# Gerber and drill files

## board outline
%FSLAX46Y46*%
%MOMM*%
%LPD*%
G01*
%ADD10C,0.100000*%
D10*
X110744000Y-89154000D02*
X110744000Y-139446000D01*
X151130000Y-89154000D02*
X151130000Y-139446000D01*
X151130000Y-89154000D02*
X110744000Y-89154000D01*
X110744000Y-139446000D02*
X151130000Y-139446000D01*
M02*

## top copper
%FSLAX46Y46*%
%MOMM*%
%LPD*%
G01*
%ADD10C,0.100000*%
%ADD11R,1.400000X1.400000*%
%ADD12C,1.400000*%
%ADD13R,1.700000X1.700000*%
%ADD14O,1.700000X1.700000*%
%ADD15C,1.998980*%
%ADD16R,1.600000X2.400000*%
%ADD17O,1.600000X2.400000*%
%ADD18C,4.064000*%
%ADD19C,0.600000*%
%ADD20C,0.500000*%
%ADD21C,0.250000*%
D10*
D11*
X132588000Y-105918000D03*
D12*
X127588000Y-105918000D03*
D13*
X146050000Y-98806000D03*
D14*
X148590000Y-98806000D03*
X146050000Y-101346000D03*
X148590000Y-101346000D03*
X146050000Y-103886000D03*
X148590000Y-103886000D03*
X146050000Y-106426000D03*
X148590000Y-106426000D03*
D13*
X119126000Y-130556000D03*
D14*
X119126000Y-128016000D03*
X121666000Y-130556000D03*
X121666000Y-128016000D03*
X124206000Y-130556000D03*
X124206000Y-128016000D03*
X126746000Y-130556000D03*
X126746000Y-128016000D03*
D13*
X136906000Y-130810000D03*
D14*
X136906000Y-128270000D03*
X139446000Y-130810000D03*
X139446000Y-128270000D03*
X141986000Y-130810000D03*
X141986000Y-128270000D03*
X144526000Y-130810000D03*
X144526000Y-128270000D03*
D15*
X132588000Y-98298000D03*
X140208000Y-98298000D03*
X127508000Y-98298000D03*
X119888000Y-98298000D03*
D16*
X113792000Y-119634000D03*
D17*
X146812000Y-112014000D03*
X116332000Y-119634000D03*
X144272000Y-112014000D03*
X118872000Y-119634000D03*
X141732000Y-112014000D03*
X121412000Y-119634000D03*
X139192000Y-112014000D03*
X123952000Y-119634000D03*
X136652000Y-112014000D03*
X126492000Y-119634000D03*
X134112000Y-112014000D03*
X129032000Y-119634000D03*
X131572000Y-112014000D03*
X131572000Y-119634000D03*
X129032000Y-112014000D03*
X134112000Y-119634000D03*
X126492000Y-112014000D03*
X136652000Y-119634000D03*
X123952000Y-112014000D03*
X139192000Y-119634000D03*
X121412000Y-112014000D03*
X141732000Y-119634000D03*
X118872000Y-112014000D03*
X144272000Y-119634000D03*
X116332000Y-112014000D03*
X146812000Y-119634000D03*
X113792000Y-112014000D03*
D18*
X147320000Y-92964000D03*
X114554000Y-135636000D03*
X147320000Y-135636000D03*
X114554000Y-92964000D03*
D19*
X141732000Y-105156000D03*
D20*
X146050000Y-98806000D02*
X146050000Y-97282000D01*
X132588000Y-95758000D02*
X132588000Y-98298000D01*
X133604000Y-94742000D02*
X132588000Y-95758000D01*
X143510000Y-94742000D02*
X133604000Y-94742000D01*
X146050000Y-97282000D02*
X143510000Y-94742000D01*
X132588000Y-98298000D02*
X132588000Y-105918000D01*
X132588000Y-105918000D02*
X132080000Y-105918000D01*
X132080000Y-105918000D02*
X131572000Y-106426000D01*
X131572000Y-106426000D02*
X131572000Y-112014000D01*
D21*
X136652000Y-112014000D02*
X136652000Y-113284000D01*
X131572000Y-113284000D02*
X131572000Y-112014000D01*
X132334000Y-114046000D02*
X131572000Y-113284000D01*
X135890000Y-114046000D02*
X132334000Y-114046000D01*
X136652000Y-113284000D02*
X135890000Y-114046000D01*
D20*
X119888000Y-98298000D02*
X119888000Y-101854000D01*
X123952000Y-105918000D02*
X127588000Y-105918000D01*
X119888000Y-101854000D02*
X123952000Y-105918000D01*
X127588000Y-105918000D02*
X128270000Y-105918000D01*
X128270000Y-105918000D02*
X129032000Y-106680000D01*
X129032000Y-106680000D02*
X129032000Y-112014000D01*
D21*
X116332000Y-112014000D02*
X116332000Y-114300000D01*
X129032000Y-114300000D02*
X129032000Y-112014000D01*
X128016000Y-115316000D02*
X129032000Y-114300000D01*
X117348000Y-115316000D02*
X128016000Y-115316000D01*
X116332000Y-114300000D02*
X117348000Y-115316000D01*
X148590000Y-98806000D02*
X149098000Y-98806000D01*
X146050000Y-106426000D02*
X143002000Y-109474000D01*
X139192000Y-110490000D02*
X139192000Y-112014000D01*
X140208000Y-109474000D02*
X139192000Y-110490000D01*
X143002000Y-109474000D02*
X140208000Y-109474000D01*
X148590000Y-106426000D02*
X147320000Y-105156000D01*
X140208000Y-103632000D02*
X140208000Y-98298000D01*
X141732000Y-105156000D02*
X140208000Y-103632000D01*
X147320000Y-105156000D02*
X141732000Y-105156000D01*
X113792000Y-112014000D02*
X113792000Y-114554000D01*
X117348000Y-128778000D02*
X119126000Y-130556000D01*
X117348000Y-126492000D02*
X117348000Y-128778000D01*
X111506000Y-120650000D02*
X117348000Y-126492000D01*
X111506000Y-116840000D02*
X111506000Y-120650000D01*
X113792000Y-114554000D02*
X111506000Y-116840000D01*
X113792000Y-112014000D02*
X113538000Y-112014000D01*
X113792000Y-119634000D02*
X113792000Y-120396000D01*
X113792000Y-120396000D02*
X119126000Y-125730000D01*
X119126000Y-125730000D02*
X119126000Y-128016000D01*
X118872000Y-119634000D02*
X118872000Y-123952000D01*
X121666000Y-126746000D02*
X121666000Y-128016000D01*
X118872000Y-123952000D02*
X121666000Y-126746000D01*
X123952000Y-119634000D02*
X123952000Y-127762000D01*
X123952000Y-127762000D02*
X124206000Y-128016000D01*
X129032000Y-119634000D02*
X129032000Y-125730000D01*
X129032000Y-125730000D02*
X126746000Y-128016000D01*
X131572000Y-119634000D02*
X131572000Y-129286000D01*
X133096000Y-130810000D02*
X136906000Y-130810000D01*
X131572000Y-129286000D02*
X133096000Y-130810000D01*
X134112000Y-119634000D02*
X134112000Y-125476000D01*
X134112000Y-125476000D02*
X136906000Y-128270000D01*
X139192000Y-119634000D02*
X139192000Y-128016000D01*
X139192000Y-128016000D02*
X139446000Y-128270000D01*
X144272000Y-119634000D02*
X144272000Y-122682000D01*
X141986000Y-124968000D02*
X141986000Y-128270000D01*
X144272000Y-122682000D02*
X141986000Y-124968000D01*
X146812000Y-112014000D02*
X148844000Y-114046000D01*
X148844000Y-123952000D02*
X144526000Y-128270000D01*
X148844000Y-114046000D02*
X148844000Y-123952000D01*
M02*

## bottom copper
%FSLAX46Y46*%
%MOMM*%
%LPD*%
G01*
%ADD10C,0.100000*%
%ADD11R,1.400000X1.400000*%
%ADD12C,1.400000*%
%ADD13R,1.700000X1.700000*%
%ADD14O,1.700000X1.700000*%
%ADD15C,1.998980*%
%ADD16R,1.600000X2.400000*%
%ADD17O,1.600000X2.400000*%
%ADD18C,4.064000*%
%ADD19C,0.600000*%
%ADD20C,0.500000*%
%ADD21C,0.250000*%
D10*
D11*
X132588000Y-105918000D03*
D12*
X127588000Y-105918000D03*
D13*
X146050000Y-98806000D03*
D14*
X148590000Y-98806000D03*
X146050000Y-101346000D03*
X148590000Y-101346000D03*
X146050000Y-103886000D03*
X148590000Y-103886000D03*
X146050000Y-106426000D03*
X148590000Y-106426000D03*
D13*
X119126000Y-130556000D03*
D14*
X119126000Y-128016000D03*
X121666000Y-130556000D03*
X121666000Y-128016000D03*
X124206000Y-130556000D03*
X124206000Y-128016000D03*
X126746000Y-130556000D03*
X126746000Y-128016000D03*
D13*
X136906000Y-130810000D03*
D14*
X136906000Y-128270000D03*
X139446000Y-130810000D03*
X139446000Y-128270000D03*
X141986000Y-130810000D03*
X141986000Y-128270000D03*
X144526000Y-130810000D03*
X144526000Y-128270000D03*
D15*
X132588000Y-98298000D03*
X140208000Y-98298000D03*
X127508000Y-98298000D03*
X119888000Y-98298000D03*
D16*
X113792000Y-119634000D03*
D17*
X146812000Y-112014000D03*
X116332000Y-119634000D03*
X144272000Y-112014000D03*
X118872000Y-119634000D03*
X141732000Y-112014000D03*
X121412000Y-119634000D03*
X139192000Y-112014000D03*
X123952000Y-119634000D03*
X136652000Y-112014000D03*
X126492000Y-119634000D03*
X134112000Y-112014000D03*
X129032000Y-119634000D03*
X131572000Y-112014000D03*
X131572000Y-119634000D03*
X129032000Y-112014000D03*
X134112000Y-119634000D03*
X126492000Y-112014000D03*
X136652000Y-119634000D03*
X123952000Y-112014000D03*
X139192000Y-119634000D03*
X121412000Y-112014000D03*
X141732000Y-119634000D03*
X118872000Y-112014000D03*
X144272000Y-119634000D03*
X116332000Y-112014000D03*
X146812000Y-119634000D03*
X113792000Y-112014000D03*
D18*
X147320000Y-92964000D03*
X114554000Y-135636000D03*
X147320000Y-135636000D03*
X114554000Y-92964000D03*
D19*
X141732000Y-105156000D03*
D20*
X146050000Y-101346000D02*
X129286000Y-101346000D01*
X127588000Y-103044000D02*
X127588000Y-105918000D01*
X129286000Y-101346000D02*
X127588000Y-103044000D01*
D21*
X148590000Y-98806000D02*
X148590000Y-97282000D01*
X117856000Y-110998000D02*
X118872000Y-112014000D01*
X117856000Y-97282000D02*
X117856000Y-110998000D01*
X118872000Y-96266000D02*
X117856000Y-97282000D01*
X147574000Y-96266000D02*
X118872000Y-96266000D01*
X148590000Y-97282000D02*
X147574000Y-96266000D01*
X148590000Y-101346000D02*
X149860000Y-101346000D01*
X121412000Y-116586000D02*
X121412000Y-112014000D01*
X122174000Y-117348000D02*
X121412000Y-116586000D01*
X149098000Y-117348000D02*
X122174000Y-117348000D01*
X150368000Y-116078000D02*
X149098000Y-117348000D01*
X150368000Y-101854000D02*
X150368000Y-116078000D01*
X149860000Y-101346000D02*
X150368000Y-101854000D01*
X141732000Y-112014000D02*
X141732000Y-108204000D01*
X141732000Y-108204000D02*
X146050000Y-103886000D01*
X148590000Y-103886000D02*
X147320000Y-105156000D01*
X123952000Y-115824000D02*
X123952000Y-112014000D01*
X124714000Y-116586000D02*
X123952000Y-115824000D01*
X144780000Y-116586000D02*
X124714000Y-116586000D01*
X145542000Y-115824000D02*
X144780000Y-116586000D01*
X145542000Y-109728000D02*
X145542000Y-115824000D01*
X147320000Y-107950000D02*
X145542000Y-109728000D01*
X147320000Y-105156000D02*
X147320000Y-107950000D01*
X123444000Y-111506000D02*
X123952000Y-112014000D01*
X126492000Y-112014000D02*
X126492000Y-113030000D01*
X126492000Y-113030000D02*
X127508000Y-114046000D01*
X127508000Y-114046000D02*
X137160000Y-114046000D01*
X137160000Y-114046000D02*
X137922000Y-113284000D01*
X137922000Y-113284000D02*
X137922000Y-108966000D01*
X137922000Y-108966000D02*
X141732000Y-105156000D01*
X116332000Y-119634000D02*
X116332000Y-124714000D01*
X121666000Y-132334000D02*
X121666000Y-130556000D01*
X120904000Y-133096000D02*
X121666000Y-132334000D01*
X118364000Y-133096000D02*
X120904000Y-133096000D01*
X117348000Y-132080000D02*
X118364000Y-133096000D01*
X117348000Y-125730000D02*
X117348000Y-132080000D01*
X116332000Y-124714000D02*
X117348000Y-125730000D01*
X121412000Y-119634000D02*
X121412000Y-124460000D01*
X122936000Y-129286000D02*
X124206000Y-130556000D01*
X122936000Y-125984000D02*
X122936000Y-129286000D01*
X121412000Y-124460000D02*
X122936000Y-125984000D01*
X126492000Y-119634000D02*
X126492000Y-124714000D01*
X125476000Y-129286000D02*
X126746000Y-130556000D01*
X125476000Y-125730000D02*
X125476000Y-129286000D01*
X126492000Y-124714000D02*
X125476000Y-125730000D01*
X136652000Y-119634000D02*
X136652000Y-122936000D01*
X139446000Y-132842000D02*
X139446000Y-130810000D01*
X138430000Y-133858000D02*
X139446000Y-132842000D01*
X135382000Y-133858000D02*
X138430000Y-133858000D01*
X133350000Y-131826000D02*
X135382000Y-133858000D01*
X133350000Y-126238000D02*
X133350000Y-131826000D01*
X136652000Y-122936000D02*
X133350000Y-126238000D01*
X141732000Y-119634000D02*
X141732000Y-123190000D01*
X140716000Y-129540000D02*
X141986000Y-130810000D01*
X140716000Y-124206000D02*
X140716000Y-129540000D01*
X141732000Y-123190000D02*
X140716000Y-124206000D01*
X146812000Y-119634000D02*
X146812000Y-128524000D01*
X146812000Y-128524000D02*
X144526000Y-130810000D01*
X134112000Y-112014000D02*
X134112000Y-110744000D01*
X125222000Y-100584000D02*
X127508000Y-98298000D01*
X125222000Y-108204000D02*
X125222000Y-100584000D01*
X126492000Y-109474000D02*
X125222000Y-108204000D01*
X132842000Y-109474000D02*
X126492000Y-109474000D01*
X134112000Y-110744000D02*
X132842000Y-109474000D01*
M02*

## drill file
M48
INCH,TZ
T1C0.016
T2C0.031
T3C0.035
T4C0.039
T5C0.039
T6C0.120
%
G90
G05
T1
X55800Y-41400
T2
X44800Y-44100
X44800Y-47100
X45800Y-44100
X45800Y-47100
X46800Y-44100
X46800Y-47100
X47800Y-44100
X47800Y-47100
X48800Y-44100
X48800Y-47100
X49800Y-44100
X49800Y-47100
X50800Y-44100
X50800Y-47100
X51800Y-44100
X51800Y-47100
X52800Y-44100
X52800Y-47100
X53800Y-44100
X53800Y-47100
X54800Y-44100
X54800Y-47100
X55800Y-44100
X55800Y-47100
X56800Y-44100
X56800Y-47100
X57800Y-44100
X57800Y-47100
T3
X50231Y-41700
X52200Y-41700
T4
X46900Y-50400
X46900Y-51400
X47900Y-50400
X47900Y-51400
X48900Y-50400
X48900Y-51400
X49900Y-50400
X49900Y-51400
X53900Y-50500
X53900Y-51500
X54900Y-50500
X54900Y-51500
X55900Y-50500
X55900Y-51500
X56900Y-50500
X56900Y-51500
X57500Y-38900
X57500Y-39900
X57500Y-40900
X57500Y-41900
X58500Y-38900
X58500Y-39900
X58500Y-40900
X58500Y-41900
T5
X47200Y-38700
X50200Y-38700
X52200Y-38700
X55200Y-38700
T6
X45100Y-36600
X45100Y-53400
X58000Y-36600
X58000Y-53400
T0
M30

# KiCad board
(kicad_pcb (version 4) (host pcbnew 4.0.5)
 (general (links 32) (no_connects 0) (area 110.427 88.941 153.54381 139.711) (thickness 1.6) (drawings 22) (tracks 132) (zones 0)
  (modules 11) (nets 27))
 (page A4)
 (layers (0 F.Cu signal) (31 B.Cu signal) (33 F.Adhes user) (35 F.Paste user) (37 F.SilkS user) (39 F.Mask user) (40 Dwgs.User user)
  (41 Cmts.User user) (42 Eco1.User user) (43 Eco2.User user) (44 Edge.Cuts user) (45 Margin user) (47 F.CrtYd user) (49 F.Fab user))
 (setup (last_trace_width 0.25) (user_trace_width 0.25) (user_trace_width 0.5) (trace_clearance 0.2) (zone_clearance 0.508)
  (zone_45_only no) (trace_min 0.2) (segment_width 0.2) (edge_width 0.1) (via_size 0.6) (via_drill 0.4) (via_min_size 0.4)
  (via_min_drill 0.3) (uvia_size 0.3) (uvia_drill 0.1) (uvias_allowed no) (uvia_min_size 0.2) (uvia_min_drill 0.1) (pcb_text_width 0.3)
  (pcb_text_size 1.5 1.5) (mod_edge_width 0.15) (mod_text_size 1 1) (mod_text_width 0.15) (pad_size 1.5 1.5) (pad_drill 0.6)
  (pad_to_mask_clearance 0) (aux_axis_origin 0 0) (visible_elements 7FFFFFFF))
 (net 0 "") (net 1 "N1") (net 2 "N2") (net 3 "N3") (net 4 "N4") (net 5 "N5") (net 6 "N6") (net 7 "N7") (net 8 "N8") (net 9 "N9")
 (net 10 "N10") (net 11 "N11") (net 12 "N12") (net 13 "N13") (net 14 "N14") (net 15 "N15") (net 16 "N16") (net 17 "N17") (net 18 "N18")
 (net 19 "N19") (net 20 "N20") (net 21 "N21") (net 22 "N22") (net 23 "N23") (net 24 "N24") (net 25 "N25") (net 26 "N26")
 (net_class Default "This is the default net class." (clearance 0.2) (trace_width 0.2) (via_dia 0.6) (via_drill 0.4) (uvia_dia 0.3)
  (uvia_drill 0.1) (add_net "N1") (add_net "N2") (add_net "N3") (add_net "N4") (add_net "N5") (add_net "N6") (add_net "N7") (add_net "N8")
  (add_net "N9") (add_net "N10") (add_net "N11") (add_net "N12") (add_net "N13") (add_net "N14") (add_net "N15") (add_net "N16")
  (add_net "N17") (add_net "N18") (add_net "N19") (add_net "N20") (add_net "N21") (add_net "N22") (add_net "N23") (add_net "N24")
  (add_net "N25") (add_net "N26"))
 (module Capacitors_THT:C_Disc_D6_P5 (layer F.Cu) (at 132.588 105.918 180)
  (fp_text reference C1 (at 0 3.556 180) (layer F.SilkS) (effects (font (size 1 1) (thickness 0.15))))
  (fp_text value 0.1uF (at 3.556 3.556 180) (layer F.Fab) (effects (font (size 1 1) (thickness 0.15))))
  (pad 1 thru_hole rect (at 0 0 180) (size 1.4 1.4) (drill 0.9) (layers *.Cu *.Mask) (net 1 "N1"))
  (pad 2 thru_hole circle (at 5 0 180) (size 1.4 1.4) (drill 0.9) (layers *.Cu *.Mask) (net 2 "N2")))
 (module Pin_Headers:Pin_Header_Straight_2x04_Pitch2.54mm (layer F.Cu) (at 146.05 98.806)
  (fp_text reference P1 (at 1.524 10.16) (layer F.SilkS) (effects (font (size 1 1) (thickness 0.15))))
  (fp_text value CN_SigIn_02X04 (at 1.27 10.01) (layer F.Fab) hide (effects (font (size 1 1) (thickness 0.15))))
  (pad 1 thru_hole rect (at 0 0) (size 1.7 1.7) (drill 1) (layers *.Cu *.Mask) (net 1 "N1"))
  (pad 2 thru_hole oval (at 2.54 0) (size 1.7 1.7) (drill 1) (layers *.Cu *.Mask) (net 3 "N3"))
  (pad 3 thru_hole oval (at 0 2.54) (size 1.7 1.7) (drill 1) (layers *.Cu *.Mask) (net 2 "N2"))
  (pad 4 thru_hole oval (at 2.54 2.54) (size 1.7 1.7) (drill 1) (layers *.Cu *.Mask) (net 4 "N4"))
  (pad 5 thru_hole oval (at 0 5.08) (size 1.7 1.7) (drill 1) (layers *.Cu *.Mask) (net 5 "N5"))
  (pad 6 thru_hole oval (at 2.54 5.08) (size 1.7 1.7) (drill 1) (layers *.Cu *.Mask) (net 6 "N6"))
  (pad 7 thru_hole oval (at 0 7.62) (size 1.7 1.7) (drill 1) (layers *.Cu *.Mask) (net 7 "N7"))
  (pad 8 thru_hole oval (at 2.54 7.62) (size 1.7 1.7) (drill 1) (layers *.Cu *.Mask) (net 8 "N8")))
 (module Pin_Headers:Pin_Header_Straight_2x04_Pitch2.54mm (layer F.Cu) (at 119.126 130.556 90)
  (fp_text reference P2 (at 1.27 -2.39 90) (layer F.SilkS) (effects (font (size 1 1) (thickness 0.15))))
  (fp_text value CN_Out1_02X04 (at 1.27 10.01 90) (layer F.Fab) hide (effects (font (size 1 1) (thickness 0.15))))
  (pad 1 thru_hole rect (at 0 0 90) (size 1.7 1.7) (drill 1) (layers *.Cu *.Mask) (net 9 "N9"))
  (pad 2 thru_hole oval (at 2.54 0 90) (size 1.7 1.7) (drill 1) (layers *.Cu *.Mask) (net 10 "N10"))
  (pad 3 thru_hole oval (at 0 2.54 90) (size 1.7 1.7) (drill 1) (layers *.Cu *.Mask) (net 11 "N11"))
  (pad 4 thru_hole oval (at 2.54 2.54 90) (size 1.7 1.7) (drill 1) (layers *.Cu *.Mask) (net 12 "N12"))
  (pad 5 thru_hole oval (at 0 5.08 90) (size 1.7 1.7) (drill 1) (layers *.Cu *.Mask) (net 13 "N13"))
  (pad 6 thru_hole oval (at 2.54 5.08 90) (size 1.7 1.7) (drill 1) (layers *.Cu *.Mask) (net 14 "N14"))
  (pad 7 thru_hole oval (at 0 7.62 90) (size 1.7 1.7) (drill 1) (layers *.Cu *.Mask) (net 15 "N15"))
  (pad 8 thru_hole oval (at 2.54 7.62 90) (size 1.7 1.7) (drill 1) (layers *.Cu *.Mask) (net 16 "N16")))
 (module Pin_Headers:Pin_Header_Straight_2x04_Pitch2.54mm (layer F.Cu) (at 136.906 130.81 90)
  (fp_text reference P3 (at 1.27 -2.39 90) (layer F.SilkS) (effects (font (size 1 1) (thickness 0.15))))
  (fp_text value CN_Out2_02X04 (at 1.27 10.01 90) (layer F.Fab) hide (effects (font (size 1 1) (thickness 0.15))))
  (pad 1 thru_hole rect (at 0 0 90) (size 1.7 1.7) (drill 1) (layers *.Cu *.Mask) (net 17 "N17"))
  (pad 2 thru_hole oval (at 2.54 0 90) (size 1.7 1.7) (drill 1) (layers *.Cu *.Mask) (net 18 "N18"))
  (pad 3 thru_hole oval (at 0 2.54 90) (size 1.7 1.7) (drill 1) (layers *.Cu *.Mask) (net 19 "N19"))
  (pad 4 thru_hole oval (at 2.54 2.54 90) (size 1.7 1.7) (drill 1) (layers *.Cu *.Mask) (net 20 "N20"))
  (pad 5 thru_hole oval (at 0 5.08 90) (size 1.7 1.7) (drill 1) (layers *.Cu *.Mask) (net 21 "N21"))
  (pad 6 thru_hole oval (at 2.54 5.08 90) (size 1.7 1.7) (drill 1) (layers *.Cu *.Mask) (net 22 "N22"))
  (pad 7 thru_hole oval (at 0 7.62 90) (size 1.7 1.7) (drill 1) (layers *.Cu *.Mask) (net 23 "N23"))
  (pad 8 thru_hole oval (at 2.54 7.62 90) (size 1.7 1.7) (drill 1) (layers *.Cu *.Mask) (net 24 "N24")))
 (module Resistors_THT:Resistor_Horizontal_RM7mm (layer F.Cu) (at 132.588 98.298)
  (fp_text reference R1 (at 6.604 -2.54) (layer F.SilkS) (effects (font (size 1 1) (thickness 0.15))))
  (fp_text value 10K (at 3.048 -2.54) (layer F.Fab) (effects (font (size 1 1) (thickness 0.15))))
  (pad 1 thru_hole circle (at 0 0) (size 1.99898 1.99898) (drill 1.00076) (layers *.Cu *.SilkS *.Mask) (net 1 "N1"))
  (pad 2 thru_hole circle (at 7.62 0) (size 1.99898 1.99898) (drill 1.00076) (layers *.Cu *.SilkS *.Mask) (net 8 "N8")))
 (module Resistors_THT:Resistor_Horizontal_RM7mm (layer F.Cu) (at 127.508 98.298 180)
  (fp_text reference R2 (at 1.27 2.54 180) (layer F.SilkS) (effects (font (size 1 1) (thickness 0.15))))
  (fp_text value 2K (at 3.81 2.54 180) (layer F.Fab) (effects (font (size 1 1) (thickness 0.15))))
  (pad 1 thru_hole circle (at 0 0 180) (size 1.99898 1.99898) (drill 1.00076) (layers *.Cu *.SilkS *.Mask) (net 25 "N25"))
  (pad 2 thru_hole circle (at 7.62 0 180) (size 1.99898 1.99898) (drill 1.00076) (layers *.Cu *.SilkS *.Mask) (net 2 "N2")))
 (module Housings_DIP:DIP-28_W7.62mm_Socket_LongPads (layer F.Cu) (at 113.792 119.634 90)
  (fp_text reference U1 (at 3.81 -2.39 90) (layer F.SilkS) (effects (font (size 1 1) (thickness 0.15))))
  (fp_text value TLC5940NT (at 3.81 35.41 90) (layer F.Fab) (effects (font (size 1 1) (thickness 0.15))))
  (pad 1 thru_hole rect (at 0 0 90) (size 2.4 1.6) (drill 0.8) (layers *.Cu *.Mask) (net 10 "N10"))
  (pad 15 thru_hole oval (at 7.62 33.02 90) (size 2.4 1.6) (drill 0.8) (layers *.Cu *.Mask) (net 24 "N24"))
  (pad 2 thru_hole oval (at 0 2.54 90) (size 2.4 1.6) (drill 0.8) (layers *.Cu *.Mask) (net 11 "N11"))
  (pad 16 thru_hole oval (at 7.62 30.48 90) (size 2.4 1.6) (drill 0.8) (layers *.Cu *.Mask) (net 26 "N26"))
  (pad 3 thru_hole oval (at 0 5.08 90) (size 2.4 1.6) (drill 0.8) (layers *.Cu *.Mask) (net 12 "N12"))
  (pad 17 thru_hole oval (at 7.62 27.94 90) (size 2.4 1.6) (drill 0.8) (layers *.Cu *.Mask) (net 5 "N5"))
  (pad 4 thru_hole oval (at 0 7.62 90) (size 2.4 1.6) (drill 0.8) (layers *.Cu *.Mask) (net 13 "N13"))
  (pad 18 thru_hole oval (at 7.62 25.4 90) (size 2.4 1.6) (drill 0.8) (layers *.Cu *.Mask) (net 7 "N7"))
  (pad 5 thru_hole oval (at 0 10.16 90) (size 2.4 1.6) (drill 0.8) (layers *.Cu *.Mask) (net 14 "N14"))
  (pad 19 thru_hole oval (at 7.62 22.86 90) (size 2.4 1.6) (drill 0.8) (layers *.Cu *.Mask) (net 1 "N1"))
  (pad 6 thru_hole oval (at 0 12.7 90) (size 2.4 1.6) (drill 0.8) (layers *.Cu *.Mask) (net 15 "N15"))
  (pad 20 thru_hole oval (at 7.62 20.32 90) (size 2.4 1.6) (drill 0.8) (layers *.Cu *.Mask) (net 25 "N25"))
  (pad 7 thru_hole oval (at 0 15.24 90) (size 2.4 1.6) (drill 0.8) (layers *.Cu *.Mask) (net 16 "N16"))
  (pad 21 thru_hole oval (at 7.62 17.78 90) (size 2.4 1.6) (drill 0.8) (layers *.Cu *.Mask) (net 1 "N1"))
  (pad 8 thru_hole oval (at 0 17.78 90) (size 2.4 1.6) (drill 0.8) (layers *.Cu *.Mask) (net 17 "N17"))
  (pad 22 thru_hole oval (at 7.62 15.24 90) (size 2.4 1.6) (drill 0.8) (layers *.Cu *.Mask) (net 2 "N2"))
  (pad 9 thru_hole oval (at 0 20.32 90) (size 2.4 1.6) (drill 0.8) (layers *.Cu *.Mask) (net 18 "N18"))
  (pad 23 thru_hole oval (at 7.62 12.7 90) (size 2.4 1.6) (drill 0.8) (layers *.Cu *.Mask) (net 8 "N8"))
  (pad 10 thru_hole oval (at 0 22.86 90) (size 2.4 1.6) (drill 0.8) (layers *.Cu *.Mask) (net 19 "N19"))
  (pad 24 thru_hole oval (at 7.62 10.16 90) (size 2.4 1.6) (drill 0.8) (layers *.Cu *.Mask) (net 6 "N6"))
  (pad 11 thru_hole oval (at 0 25.4 90) (size 2.4 1.6) (drill 0.8) (layers *.Cu *.Mask) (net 20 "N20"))
  (pad 25 thru_hole oval (at 7.62 7.62 90) (size 2.4 1.6) (drill 0.8) (layers *.Cu *.Mask) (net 4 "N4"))
  (pad 12 thru_hole oval (at 0 27.94 90) (size 2.4 1.6) (drill 0.8) (layers *.Cu *.Mask) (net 21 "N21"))
  (pad 26 thru_hole oval (at 7.62 5.08 90) (size 2.4 1.6) (drill 0.8) (layers *.Cu *.Mask) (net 3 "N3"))
  (pad 13 thru_hole oval (at 0 30.48 90) (size 2.4 1.6) (drill 0.8) (layers *.Cu *.Mask) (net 22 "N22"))
  (pad 27 thru_hole oval (at 7.62 2.54 90) (size 2.4 1.6) (drill 0.8) (layers *.Cu *.Mask) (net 2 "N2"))
  (pad 14 thru_hole oval (at 0 33.02 90) (size 2.4 1.6) (drill 0.8) (layers *.Cu *.Mask) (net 23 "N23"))
  (pad 28 thru_hole oval (at 7.62 0 90) (size 2.4 1.6) (drill 0.8) (layers *.Cu *.Mask) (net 9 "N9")))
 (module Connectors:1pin (layer F.Cu) (at 147.32 92.964)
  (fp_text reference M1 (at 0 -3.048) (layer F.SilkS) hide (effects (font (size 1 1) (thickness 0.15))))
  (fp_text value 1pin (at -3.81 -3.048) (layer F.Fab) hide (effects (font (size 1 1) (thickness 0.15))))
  (pad 1 thru_hole circle (at 0 0) (size 4.064 4.064) (drill 3.048) (layers *.Cu *.Mask)))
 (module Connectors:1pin (layer F.Cu) (at 114.554 135.636)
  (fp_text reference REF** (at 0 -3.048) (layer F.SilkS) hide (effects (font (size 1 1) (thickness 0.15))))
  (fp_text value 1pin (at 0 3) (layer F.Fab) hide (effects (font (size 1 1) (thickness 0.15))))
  (pad 1 thru_hole circle (at 0 0) (size 4.064 4.064) (drill 3.048) (layers *.Cu *.Mask)))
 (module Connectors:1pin (layer F.Cu) (at 147.32 135.636)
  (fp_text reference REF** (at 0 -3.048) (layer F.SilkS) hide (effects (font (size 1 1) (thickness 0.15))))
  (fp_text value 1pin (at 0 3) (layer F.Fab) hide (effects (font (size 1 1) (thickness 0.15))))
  (pad 1 thru_hole circle (at 0 0) (size 4.064 4.064) (drill 3.048) (layers *.Cu *.Mask)))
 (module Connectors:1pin (layer F.Cu) (at 114.554 92.964)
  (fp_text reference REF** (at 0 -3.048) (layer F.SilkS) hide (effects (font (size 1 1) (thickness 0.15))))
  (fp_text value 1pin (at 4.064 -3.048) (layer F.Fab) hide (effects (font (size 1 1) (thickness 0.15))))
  (pad 1 thru_hole circle (at 0 0) (size 4.064 4.064) (drill 3.048) (layers *.Cu *.Mask)))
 (gr_line (start 110.744 89.154) (end 110.744 139.446) (angle 90) (layer Edge.Cuts) (width 0.1))
 (gr_line (start 151.13 89.154) (end 151.13 139.446) (angle 90) (layer Edge.Cuts) (width 0.1))
 (gr_line (start 151.13 89.154) (end 110.744 89.154) (angle 90) (layer Edge.Cuts) (width 0.1))
 (gr_line (start 110.744 139.446) (end 151.13 139.446) (angle 90) (layer Edge.Cuts) (width 0.1))
 (segment (start 146.05 98.806) (end 146.05 97.282) (width 0.5) (layer F.Cu) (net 1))
 (segment (start 132.588 95.758) (end 132.588 98.298) (width 0.5) (layer F.Cu) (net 1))
 (segment (start 133.604 94.742) (end 132.588 95.758) (width 0.5) (layer F.Cu) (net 1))
 (segment (start 143.51 94.742) (end 133.604 94.742) (width 0.5) (layer F.Cu) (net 1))
 (segment (start 146.05 97.282) (end 143.51 94.742) (width 0.5) (layer F.Cu) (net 1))
 (segment (start 132.588 98.298) (end 132.588 105.918) (width 0.5) (layer F.Cu) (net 1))
 (segment (start 132.588 105.918) (end 132.08 105.918) (width 0.5) (layer F.Cu) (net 1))
 (segment (start 132.08 105.918) (end 131.572 106.426) (width 0.5) (layer F.Cu) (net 1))
 (segment (start 131.572 106.426) (end 131.572 112.014) (width 0.5) (layer F.Cu) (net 1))
 (segment (start 136.652 112.014) (end 136.652 113.284) (width 0.25) (layer F.Cu) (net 1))
 (segment (start 131.572 113.284) (end 131.572 112.014) (width 0.25) (layer F.Cu) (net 1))
 (segment (start 132.334 114.046) (end 131.572 113.284) (width 0.25) (layer F.Cu) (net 1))
 (segment (start 135.89 114.046) (end 132.334 114.046) (width 0.25) (layer F.Cu) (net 1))
 (segment (start 136.652 113.284) (end 135.89 114.046) (width 0.25) (layer F.Cu) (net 1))
 (segment (start 146.05 101.346) (end 129.286 101.346) (width 0.5) (layer B.Cu) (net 2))
 (segment (start 127.588 103.044) (end 127.588 105.918) (width 0.5) (layer B.Cu) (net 2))
 (segment (start 129.286 101.346) (end 127.588 103.044) (width 0.5) (layer B.Cu) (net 2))
 (segment (start 119.888 98.298) (end 119.888 101.854) (width 0.5) (layer F.Cu) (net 2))
 (segment (start 123.952 105.918) (end 127.588 105.918) (width 0.5) (layer F.Cu) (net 2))
 (segment (start 119.888 101.854) (end 123.952 105.918) (width 0.5) (layer F.Cu) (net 2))
 (segment (start 127.588 105.918) (end 128.27 105.918) (width 0.5) (layer F.Cu) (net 2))
 (segment (start 128.27 105.918) (end 129.032 106.68) (width 0.5) (layer F.Cu) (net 2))
 (segment (start 129.032 106.68) (end 129.032 112.014) (width 0.5) (layer F.Cu) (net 2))
 (segment (start 116.332 112.014) (end 116.332 114.3) (width 0.25) (layer F.Cu) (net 2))
 (segment (start 129.032 114.3) (end 129.032 112.014) (width 0.25) (layer F.Cu) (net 2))
 (segment (start 128.016 115.316) (end 129.032 114.3) (width 0.25) (layer F.Cu) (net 2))
 (segment (start 117.348 115.316) (end 128.016 115.316) (width 0.25) (layer F.Cu) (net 2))
 (segment (start 116.332 114.3) (end 117.348 115.316) (width 0.25) (layer F.Cu) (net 2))
 (segment (start 148.59 98.806) (end 148.59 97.282) (width 0.25) (layer B.Cu) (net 3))
 (segment (start 117.856 110.998) (end 118.872 112.014) (width 0.25) (layer B.Cu) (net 3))
 (segment (start 117.856 97.282) (end 117.856 110.998) (width 0.25) (layer B.Cu) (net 3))
 (segment (start 118.872 96.266) (end 117.856 97.282) (width 0.25) (layer B.Cu) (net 3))
 (segment (start 147.574 96.266) (end 118.872 96.266) (width 0.25) (layer B.Cu) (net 3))
 (segment (start 148.59 97.282) (end 147.574 96.266) (width 0.25) (layer B.Cu) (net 3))
 (segment (start 148.59 98.806) (end 149.098 98.806) (width 0.25) (layer F.Cu) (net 3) (status 30))
 (segment (start 148.59 101.346) (end 149.86 101.346) (width 0.25) (layer B.Cu) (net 4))
 (segment (start 121.412 116.586) (end 121.412 112.014) (width 0.25) (layer B.Cu) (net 4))
 (segment (start 122.174 117.348) (end 121.412 116.586) (width 0.25) (layer B.Cu) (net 4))
 (segment (start 149.098 117.348) (end 122.174 117.348) (width 0.25) (layer B.Cu) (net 4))
 (segment (start 150.368 116.078) (end 149.098 117.348) (width 0.25) (layer B.Cu) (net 4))
 (segment (start 150.368 101.854) (end 150.368 116.078) (width 0.25) (layer B.Cu) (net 4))
 (segment (start 149.86 101.346) (end 150.368 101.854) (width 0.25) (layer B.Cu) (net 4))
 (segment (start 141.732 112.014) (end 141.732 108.204) (width 0.25) (layer B.Cu) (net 5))
 (segment (start 141.732 108.204) (end 146.05 103.886) (width 0.25) (layer B.Cu) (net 5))
 (segment (start 148.59 103.886) (end 147.32 105.156) (width 0.25) (layer B.Cu) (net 6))
 (segment (start 123.952 115.824) (end 123.952 112.014) (width 0.25) (layer B.Cu) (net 6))
 (segment (start 124.714 116.586) (end 123.952 115.824) (width 0.25) (layer B.Cu) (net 6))
 (segment (start 144.78 116.586) (end 124.714 116.586) (width 0.25) (layer B.Cu) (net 6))
 (segment (start 145.542 115.824) (end 144.78 116.586) (width 0.25) (layer B.Cu) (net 6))
 (segment (start 145.542 109.728) (end 145.542 115.824) (width 0.25) (layer B.Cu) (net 6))
 (segment (start 147.32 107.95) (end 145.542 109.728) (width 0.25) (layer B.Cu) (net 6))
 (segment (start 147.32 105.156) (end 147.32 107.95) (width 0.25) (layer B.Cu) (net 6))
 (segment (start 123.444 111.506) (end 123.952 112.014) (width 0.25) (layer B.Cu) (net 6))
 (segment (start 146.05 106.426) (end 143.002 109.474) (width 0.25) (layer F.Cu) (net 7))
 (segment (start 139.192 110.49) (end 139.192 112.014) (width 0.25) (layer F.Cu) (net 7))
 (segment (start 140.208 109.474) (end 139.192 110.49) (width 0.25) (layer F.Cu) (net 7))
 (segment (start 143.002 109.474) (end 140.208 109.474) (width 0.25) (layer F.Cu) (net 7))
 (segment (start 126.492 112.014) (end 126.492 113.03) (width 0.25) (layer B.Cu) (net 8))
 (segment (start 126.492 113.03) (end 127.508 114.046) (width 0.25) (layer B.Cu) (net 8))
 (segment (start 127.508 114.046) (end 137.16 114.046) (width 0.25) (layer B.Cu) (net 8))
 (segment (start 137.16 114.046) (end 137.922 113.284) (width 0.25) (layer B.Cu) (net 8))
 (segment (start 137.922 113.284) (end 137.922 108.966) (width 0.25) (layer B.Cu) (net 8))
 (segment (start 137.922 108.966) (end 141.732 105.156) (width 0.25) (layer B.Cu) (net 8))
 (via (at 141.732 105.156) (size 0.6) (drill 0.4) (layers F.Cu B.Cu) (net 8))
 (segment (start 148.59 106.426) (end 147.32 105.156) (width 0.25) (layer F.Cu) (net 8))
 (segment (start 140.208 103.632) (end 140.208 98.298) (width 0.25) (layer F.Cu) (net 8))
 (segment (start 141.732 105.156) (end 140.208 103.632) (width 0.25) (layer F.Cu) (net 8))
 (segment (start 147.32 105.156) (end 141.732 105.156) (width 0.25) (layer F.Cu) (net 8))
 (segment (start 113.792 112.014) (end 113.792 114.554) (width 0.25) (layer F.Cu) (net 9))
 (segment (start 117.348 128.778) (end 119.126 130.556) (width 0.25) (layer F.Cu) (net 9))
 (segment (start 117.348 126.492) (end 117.348 128.778) (width 0.25) (layer F.Cu) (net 9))
 (segment (start 111.506 120.65) (end 117.348 126.492) (width 0.25) (layer F.Cu) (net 9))
 (segment (start 111.506 116.84) (end 111.506 120.65) (width 0.25) (layer F.Cu) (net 9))
 (segment (start 113.792 114.554) (end 111.506 116.84) (width 0.25) (layer F.Cu) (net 9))
 (segment (start 113.792 112.014) (end 113.538 112.014) (width 0.25) (layer F.Cu) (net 9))
 (segment (start 113.792 119.634) (end 113.792 120.396) (width 0.25) (layer F.Cu) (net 10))
 (segment (start 113.792 120.396) (end 119.126 125.73) (width 0.25) (layer F.Cu) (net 10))
 (segment (start 119.126 125.73) (end 119.126 128.016) (width 0.25) (layer F.Cu) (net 10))
 (segment (start 116.332 119.634) (end 116.332 124.714) (width 0.25) (layer B.Cu) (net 11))
 (segment (start 121.666 132.334) (end 121.666 130.556) (width 0.25) (layer B.Cu) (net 11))
 (segment (start 120.904 133.096) (end 121.666 132.334) (width 0.25) (layer B.Cu) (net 11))
 (segment (start 118.364 133.096) (end 120.904 133.096) (width 0.25) (layer B.Cu) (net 11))
 (segment (start 117.348 132.08) (end 118.364 133.096) (width 0.25) (layer B.Cu) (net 11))
 (segment (start 117.348 125.73) (end 117.348 132.08) (width 0.25) (layer B.Cu) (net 11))
 (segment (start 116.332 124.714) (end 117.348 125.73) (width 0.25) (layer B.Cu) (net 11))
 (segment (start 118.872 119.634) (end 118.872 123.952) (width 0.25) (layer F.Cu) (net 12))
 (segment (start 121.666 126.746) (end 121.666 128.016) (width 0.25) (layer F.Cu) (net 12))
 (segment (start 118.872 123.952) (end 121.666 126.746) (width 0.25) (layer F.Cu) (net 12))
 (segment (start 121.412 119.634) (end 121.412 124.46) (width 0.25) (layer B.Cu) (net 13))
 (segment (start 122.936 129.286) (end 124.206 130.556) (width 0.25) (layer B.Cu) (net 13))
 (segment (start 122.936 125.984) (end 122.936 129.286) (width 0.25) (layer B.Cu) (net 13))
 (segment (start 121.412 124.46) (end 122.936 125.984) (width 0.25) (layer B.Cu) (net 13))
 (segment (start 123.952 119.634) (end 123.952 127.762) (width 0.25) (layer F.Cu) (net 14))
 (segment (start 123.952 127.762) (end 124.206 128.016) (width 0.25) (layer F.Cu) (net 14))
 (segment (start 126.492 119.634) (end 126.492 124.714) (width 0.25) (layer B.Cu) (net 15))
 (segment (start 125.476 129.286) (end 126.746 130.556) (width 0.25) (layer B.Cu) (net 15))
 (segment (start 125.476 125.73) (end 125.476 129.286) (width 0.25) (layer B.Cu) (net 15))
 (segment (start 126.492 124.714) (end 125.476 125.73) (width 0.25) (layer B.Cu) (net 15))
 (segment (start 129.032 119.634) (end 129.032 125.73) (width 0.25) (layer F.Cu) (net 16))
 (segment (start 129.032 125.73) (end 126.746 128.016) (width 0.25) (layer F.Cu) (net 16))
 (segment (start 131.572 119.634) (end 131.572 129.286) (width 0.25) (layer F.Cu) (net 17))
 (segment (start 133.096 130.81) (end 136.906 130.81) (width 0.25) (layer F.Cu) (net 17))
 (segment (start 131.572 129.286) (end 133.096 130.81) (width 0.25) (layer F.Cu) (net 17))
 (segment (start 134.112 119.634) (end 134.112 125.476) (width 0.25) (layer F.Cu) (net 18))
 (segment (start 134.112 125.476) (end 136.906 128.27) (width 0.25) (layer F.Cu) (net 18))
 (segment (start 136.652 119.634) (end 136.652 122.936) (width 0.25) (layer B.Cu) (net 19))
 (segment (start 139.446 132.842) (end 139.446 130.81) (width 0.25) (layer B.Cu) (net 19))
 (segment (start 138.43 133.858) (end 139.446 132.842) (width 0.25) (layer B.Cu) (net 19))
 (segment (start 135.382 133.858) (end 138.43 133.858) (width 0.25) (layer B.Cu) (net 19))
 (segment (start 133.35 131.826) (end 135.382 133.858) (width 0.25) (layer B.Cu) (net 19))
 (segment (start 133.35 126.238) (end 133.35 131.826) (width 0.25) (layer B.Cu) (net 19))
 (segment (start 136.652 122.936) (end 133.35 126.238) (width 0.25) (layer B.Cu) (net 19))
 (segment (start 139.192 119.634) (end 139.192 128.016) (width 0.25) (layer F.Cu) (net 20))
 (segment (start 139.192 128.016) (end 139.446 128.27) (width 0.25) (layer F.Cu) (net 20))
 (segment (start 141.732 119.634) (end 141.732 123.19) (width 0.25) (layer B.Cu) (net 21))
 (segment (start 140.716 129.54) (end 141.986 130.81) (width 0.25) (layer B.Cu) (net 21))
 (segment (start 140.716 124.206) (end 140.716 129.54) (width 0.25) (layer B.Cu) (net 21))
 (segment (start 141.732 123.19) (end 140.716 124.206) (width 0.25) (layer B.Cu) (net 21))
 (segment (start 144.272 119.634) (end 144.272 122.682) (width 0.25) (layer F.Cu) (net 22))
 (segment (start 141.986 124.968) (end 141.986 128.27) (width 0.25) (layer F.Cu) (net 22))
 (segment (start 144.272 122.682) (end 141.986 124.968) (width 0.25) (layer F.Cu) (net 22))
 (segment (start 146.812 119.634) (end 146.812 128.524) (width 0.25) (layer B.Cu) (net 23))
 (segment (start 146.812 128.524) (end 144.526 130.81) (width 0.25) (layer B.Cu) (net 23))
 (segment (start 146.812 112.014) (end 148.844 114.046) (width 0.25) (layer F.Cu) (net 24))
 (segment (start 148.844 123.952) (end 144.526 128.27) (width 0.25) (layer F.Cu) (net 24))
 (segment (start 148.844 114.046) (end 148.844 123.952) (width 0.25) (layer F.Cu) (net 24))
 (segment (start 134.112 112.014) (end 134.112 110.744) (width 0.25) (layer B.Cu) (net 25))
 (segment (start 125.222 100.584) (end 127.508 98.298) (width 0.25) (layer B.Cu) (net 25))
 (segment (start 125.222 108.204) (end 125.222 100.584) (width 0.25) (layer B.Cu) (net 25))
 (segment (start 126.492 109.474) (end 125.222 108.204) (width 0.25) (layer B.Cu) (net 25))
 (segment (start 132.842 109.474) (end 126.492 109.474) (width 0.25) (layer B.Cu) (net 25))
 (segment (start 134.112 110.744) (end 132.842 109.474) (width 0.25) (layer B.Cu) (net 25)))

